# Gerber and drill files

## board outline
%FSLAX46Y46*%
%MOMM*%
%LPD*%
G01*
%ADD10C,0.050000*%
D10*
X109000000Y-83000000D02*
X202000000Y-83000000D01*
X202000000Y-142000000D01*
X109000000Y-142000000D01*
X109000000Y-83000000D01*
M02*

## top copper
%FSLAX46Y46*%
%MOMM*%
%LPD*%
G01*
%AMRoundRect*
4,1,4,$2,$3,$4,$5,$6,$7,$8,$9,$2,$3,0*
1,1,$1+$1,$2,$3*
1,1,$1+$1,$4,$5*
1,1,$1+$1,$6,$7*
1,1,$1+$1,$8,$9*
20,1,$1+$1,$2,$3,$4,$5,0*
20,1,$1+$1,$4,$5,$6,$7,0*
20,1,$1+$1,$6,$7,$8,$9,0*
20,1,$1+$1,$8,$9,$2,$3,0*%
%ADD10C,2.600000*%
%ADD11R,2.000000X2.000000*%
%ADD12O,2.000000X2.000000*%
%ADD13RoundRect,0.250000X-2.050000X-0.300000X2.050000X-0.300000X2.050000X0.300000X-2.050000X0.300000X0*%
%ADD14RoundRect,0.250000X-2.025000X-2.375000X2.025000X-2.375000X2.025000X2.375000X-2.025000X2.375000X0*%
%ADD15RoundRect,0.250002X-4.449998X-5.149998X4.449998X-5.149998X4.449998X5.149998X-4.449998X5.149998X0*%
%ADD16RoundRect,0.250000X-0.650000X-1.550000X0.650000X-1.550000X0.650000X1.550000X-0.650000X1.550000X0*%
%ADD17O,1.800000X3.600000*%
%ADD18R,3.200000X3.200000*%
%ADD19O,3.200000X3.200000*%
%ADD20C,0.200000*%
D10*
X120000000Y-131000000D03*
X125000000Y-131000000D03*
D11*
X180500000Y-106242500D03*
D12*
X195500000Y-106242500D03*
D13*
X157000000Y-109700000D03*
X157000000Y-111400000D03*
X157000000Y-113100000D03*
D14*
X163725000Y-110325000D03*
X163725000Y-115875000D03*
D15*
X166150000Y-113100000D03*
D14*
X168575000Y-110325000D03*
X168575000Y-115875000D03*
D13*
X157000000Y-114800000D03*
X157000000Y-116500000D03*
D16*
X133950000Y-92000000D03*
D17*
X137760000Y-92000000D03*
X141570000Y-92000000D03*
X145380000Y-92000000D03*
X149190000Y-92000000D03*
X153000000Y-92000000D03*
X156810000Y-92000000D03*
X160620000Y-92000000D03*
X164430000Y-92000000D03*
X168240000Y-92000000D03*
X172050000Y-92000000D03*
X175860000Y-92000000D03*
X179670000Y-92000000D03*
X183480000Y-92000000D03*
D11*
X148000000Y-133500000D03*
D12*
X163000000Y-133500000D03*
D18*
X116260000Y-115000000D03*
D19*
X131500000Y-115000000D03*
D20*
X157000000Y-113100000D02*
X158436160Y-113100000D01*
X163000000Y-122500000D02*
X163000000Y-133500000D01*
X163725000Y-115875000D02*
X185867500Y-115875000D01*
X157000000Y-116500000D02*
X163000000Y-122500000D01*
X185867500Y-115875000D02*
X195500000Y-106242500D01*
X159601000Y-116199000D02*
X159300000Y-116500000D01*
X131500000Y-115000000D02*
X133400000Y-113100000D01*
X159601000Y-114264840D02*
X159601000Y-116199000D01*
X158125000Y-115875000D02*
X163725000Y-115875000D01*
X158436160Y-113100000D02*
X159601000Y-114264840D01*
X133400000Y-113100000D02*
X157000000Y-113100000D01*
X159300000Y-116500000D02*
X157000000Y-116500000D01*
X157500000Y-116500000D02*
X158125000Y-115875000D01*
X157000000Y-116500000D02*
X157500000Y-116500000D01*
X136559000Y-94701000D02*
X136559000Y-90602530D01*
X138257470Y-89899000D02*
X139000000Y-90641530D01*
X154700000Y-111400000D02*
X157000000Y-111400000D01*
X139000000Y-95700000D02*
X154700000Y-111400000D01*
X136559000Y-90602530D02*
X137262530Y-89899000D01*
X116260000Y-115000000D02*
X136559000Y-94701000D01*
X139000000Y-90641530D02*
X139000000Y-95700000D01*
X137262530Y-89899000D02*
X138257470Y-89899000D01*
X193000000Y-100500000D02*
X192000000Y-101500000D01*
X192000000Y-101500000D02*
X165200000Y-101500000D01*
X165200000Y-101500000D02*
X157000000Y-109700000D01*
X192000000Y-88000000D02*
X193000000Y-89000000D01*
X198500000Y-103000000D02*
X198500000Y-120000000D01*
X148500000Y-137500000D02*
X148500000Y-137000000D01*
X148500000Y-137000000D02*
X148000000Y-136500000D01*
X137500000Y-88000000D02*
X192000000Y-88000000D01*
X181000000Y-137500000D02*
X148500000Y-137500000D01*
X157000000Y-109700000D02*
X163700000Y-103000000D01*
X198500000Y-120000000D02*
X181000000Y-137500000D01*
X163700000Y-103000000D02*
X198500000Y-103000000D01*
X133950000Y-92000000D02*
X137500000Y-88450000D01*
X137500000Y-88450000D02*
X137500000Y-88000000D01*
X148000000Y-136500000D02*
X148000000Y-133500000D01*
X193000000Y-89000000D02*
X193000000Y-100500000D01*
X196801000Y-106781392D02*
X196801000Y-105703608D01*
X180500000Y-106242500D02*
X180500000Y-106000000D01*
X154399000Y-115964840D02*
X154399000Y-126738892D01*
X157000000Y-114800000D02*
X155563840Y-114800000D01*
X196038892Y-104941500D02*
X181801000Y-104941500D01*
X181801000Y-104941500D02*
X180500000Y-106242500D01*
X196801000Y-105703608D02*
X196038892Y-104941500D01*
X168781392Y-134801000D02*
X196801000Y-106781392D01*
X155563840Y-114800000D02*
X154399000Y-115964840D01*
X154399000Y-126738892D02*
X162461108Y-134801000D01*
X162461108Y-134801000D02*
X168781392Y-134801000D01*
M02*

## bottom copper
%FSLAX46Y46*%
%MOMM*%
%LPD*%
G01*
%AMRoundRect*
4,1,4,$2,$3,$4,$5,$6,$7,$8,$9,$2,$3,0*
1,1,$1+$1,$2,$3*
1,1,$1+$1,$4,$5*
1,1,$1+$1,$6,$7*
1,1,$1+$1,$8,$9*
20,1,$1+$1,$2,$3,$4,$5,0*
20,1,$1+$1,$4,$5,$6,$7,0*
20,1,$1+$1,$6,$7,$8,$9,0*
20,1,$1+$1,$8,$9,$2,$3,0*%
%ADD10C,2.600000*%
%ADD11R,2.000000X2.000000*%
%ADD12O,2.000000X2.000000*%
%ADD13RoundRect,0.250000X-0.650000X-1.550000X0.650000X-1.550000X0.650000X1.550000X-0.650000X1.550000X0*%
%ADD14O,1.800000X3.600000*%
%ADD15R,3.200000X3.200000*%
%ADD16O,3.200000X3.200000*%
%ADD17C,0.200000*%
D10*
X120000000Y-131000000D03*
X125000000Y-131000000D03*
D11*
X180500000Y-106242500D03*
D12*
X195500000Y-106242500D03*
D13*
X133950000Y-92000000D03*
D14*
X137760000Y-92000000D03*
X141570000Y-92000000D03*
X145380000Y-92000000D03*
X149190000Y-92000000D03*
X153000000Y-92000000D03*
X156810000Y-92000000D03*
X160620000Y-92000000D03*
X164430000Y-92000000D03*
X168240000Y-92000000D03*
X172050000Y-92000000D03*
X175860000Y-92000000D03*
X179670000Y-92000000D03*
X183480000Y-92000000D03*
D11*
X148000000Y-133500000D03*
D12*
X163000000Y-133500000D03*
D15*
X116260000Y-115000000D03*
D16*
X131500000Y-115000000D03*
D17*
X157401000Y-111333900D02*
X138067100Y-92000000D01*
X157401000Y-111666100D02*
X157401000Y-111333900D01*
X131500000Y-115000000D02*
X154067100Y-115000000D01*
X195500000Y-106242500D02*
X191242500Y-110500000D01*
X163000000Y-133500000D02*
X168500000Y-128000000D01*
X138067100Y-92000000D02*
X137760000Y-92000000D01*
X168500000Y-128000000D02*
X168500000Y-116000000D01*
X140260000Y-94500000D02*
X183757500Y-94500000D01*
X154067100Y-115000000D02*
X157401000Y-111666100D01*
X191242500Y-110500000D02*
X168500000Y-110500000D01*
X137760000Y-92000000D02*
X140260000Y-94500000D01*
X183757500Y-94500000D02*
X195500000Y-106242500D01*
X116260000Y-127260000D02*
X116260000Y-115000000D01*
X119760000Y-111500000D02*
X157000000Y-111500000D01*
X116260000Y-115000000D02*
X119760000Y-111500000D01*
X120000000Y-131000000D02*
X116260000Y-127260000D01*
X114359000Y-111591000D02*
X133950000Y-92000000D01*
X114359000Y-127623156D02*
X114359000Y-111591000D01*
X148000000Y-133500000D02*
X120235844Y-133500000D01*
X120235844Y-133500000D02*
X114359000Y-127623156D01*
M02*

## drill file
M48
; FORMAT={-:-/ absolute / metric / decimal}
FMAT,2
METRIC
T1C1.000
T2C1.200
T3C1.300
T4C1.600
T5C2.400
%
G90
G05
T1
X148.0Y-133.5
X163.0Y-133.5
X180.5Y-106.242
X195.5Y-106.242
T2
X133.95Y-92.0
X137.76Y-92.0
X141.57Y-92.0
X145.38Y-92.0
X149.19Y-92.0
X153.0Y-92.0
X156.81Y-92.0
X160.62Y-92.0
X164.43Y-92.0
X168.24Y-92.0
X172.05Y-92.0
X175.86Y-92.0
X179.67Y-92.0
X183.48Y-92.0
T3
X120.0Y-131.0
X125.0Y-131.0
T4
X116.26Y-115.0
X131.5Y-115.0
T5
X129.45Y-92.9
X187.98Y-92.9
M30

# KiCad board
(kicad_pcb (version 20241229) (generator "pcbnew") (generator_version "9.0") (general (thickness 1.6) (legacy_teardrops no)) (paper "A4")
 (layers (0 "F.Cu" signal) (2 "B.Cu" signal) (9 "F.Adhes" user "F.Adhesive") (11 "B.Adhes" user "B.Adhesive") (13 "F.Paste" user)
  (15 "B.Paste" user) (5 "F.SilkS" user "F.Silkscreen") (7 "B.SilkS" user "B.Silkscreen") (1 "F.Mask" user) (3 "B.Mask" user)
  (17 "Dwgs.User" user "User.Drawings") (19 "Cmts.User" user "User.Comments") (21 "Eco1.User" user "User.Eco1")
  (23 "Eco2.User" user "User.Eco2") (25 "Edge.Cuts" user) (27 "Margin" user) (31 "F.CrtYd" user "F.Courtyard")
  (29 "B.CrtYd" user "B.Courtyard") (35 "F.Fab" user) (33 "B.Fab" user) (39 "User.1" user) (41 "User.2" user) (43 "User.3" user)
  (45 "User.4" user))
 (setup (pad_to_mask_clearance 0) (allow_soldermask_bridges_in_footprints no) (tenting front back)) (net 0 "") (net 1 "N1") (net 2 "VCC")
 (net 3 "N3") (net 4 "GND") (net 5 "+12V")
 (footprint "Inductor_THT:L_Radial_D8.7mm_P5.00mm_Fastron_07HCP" (layer "F.Cu") (at 120 131)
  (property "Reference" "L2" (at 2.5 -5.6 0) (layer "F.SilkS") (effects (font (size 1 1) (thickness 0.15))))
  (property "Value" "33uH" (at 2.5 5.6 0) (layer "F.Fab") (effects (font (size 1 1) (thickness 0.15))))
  (pad "1" thru_hole circle (at 0 0) (size 2.6 2.6) (drill 1.3) (layers "*.Cu" "*.Mask") (remove_unused_layers no) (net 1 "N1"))
  (pad "2" thru_hole circle (at 5 0) (size 2.6 2.6) (drill 1.3) (layers "*.Cu" "*.Mask") (remove_unused_layers no) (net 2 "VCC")))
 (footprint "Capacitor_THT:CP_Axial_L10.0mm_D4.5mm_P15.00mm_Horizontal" (layer "F.Cu") (at 180.5 106.2425)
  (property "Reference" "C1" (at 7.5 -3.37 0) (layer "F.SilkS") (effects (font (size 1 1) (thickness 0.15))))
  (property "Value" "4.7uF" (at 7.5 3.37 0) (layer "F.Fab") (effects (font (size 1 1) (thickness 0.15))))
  (pad "1" thru_hole rect (at 0 0) (size 2 2) (drill 1) (layers "*.Cu" "*.Mask") (remove_unused_layers no) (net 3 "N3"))
  (pad "2" thru_hole oval (at 15 0) (size 2 2) (drill 1) (layers "*.Cu" "*.Mask") (remove_unused_layers no) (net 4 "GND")))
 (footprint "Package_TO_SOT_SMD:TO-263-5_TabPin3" (layer "F.Cu") (at 164.65 113.1)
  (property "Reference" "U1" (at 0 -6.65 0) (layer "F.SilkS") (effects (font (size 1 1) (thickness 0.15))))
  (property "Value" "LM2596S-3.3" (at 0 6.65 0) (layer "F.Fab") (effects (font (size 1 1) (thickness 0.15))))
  (pad "1" smd roundrect (at -7.65 -3.4) (size 4.6 1.1) (layers "F.Cu" "F.Mask" "F.Paste") (roundrect_rratio 0.227273) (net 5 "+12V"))
  (pad "2" smd roundrect (at -7.65 -1.7) (size 4.6 1.1) (layers "F.Cu" "F.Mask" "F.Paste") (roundrect_rratio 0.227273) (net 1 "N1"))
  (pad "3" smd roundrect (at -7.65 0) (size 4.6 1.1) (layers "F.Cu" "F.Mask" "F.Paste") (roundrect_rratio 0.227273) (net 4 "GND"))
  (pad "3" smd roundrect (at -0.925 -2.775) (size 4.55 5.25) (layers "F.Cu" "F.Paste") (roundrect_rratio 0.054945) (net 4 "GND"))
  (pad "3" smd roundrect (at -0.925 2.775) (size 4.55 5.25) (layers "F.Cu" "F.Paste") (roundrect_rratio 0.054945) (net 4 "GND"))
  (pad "3" smd roundrect (at 1.5 0) (size 9.4 10.8) (layers "F.Cu" "F.Mask") (roundrect_rratio 0.026596) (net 4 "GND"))
  (pad "3" smd roundrect (at 3.925 -2.775) (size 4.55 5.25) (layers "F.Cu" "F.Paste") (roundrect_rratio 0.054945) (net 4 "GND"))
  (pad "3" smd roundrect (at 3.925 2.775) (size 4.55 5.25) (layers "F.Cu" "F.Paste") (roundrect_rratio 0.054945) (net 4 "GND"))
  (pad "4" smd roundrect (at -7.65 1.7) (size 4.6 1.1) (layers "F.Cu" "F.Mask" "F.Paste") (roundrect_rratio 0.227273) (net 3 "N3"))
  (pad "5" smd roundrect (at -7.65 3.4) (size 4.6 1.1) (layers "F.Cu" "F.Mask" "F.Paste") (roundrect_rratio 0.227273) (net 4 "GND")))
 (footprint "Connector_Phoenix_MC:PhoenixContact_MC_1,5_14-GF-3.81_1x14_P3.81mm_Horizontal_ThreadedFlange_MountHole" (layer "F.Cu")
  (at 133.95 92)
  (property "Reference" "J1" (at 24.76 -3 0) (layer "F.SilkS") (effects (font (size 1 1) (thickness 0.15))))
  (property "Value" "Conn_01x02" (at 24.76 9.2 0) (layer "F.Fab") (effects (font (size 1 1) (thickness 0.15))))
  (pad "" np_thru_hole circle (at -4.5 0.9) (size 2.4 2.4) (drill 2.4) (layers "*.Cu" "*.Mask"))
  (pad "" np_thru_hole circle (at 54.03 0.9) (size 2.4 2.4) (drill 2.4) (layers "*.Cu" "*.Mask"))
  (pad "1" thru_hole roundrect (at 0 0) (size 1.8 3.6) (drill 1.2) (layers "*.Cu" "*.Mask") (remove_unused_layers no)
   (roundrect_rratio 0.138889) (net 5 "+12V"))
  (pad "2" thru_hole oval (at 3.81 0) (size 1.8 3.6) (drill 1.2) (layers "*.Cu" "*.Mask") (remove_unused_layers no) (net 4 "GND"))
  (pad "3" thru_hole oval (at 7.62 0) (size 1.8 3.6) (drill 1.2) (layers "*.Cu" "*.Mask") (remove_unused_layers no))
  (pad "4" thru_hole oval (at 11.43 0) (size 1.8 3.6) (drill 1.2) (layers "*.Cu" "*.Mask") (remove_unused_layers no))
  (pad "5" thru_hole oval (at 15.24 0) (size 1.8 3.6) (drill 1.2) (layers "*.Cu" "*.Mask") (remove_unused_layers no))
  (pad "6" thru_hole oval (at 19.05 0) (size 1.8 3.6) (drill 1.2) (layers "*.Cu" "*.Mask") (remove_unused_layers no))
  (pad "7" thru_hole oval (at 22.86 0) (size 1.8 3.6) (drill 1.2) (layers "*.Cu" "*.Mask") (remove_unused_layers no))
  (pad "8" thru_hole oval (at 26.67 0) (size 1.8 3.6) (drill 1.2) (layers "*.Cu" "*.Mask") (remove_unused_layers no))
  (pad "9" thru_hole oval (at 30.48 0) (size 1.8 3.6) (drill 1.2) (layers "*.Cu" "*.Mask") (remove_unused_layers no))
  (pad "10" thru_hole oval (at 34.29 0) (size 1.8 3.6) (drill 1.2) (layers "*.Cu" "*.Mask") (remove_unused_layers no))
  (pad "11" thru_hole oval (at 38.1 0) (size 1.8 3.6) (drill 1.2) (layers "*.Cu" "*.Mask") (remove_unused_layers no))
  (pad "12" thru_hole oval (at 41.91 0) (size 1.8 3.6) (drill 1.2) (layers "*.Cu" "*.Mask") (remove_unused_layers no))
  (pad "13" thru_hole oval (at 45.72 0) (size 1.8 3.6) (drill 1.2) (layers "*.Cu" "*.Mask") (remove_unused_layers no))
  (pad "14" thru_hole oval (at 49.53 0) (size 1.8 3.6) (drill 1.2) (layers "*.Cu" "*.Mask") (remove_unused_layers no)))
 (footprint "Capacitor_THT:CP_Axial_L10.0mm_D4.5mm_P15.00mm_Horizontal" (layer "F.Cu") (at 148 133.5)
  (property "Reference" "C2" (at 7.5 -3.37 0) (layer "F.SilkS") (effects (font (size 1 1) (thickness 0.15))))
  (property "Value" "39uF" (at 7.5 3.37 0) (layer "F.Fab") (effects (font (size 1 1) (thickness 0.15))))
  (pad "1" thru_hole rect (at 0 0) (size 2 2) (drill 1) (layers "*.Cu" "*.Mask") (remove_unused_layers no) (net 5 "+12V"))
  (pad "2" thru_hole oval (at 15 0) (size 2 2) (drill 1) (layers "*.Cu" "*.Mask") (remove_unused_layers no) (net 4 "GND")))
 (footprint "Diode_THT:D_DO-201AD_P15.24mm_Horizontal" (layer "F.Cu") (at 116.26 115)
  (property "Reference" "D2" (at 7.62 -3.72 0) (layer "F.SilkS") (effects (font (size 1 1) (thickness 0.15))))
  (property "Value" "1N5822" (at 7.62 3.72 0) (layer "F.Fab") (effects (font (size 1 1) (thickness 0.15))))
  (pad "1" thru_hole rect (at 0 0) (size 3.2 3.2) (drill 1.6) (layers "*.Cu" "*.Mask") (remove_unused_layers no) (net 1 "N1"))
  (pad "2" thru_hole oval (at 15.24 0) (size 3.2 3.2) (drill 1.6) (layers "*.Cu" "*.Mask") (remove_unused_layers no) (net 4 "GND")))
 (gr_rect (start 109 83) (end 202 142) (stroke (width 0.05) (type default)) (fill no) (layer "Edge.Cuts"))
 (segment (start 157 113.1) (end 158.43616 113.1) (width 0.2) (layer "F.Cu") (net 4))
 (segment (start 163 122.5) (end 163 133.5) (width 0.2) (layer "F.Cu") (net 4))
 (segment (start 163.725 115.875) (end 185.8675 115.875) (width 0.2) (layer "F.Cu") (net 4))
 (segment (start 157 116.5) (end 163 122.5) (width 0.2) (layer "F.Cu") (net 4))
 (segment (start 185.8675 115.875) (end 195.5 106.2425) (width 0.2) (layer "F.Cu") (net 4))
 (segment (start 159.601 116.199) (end 159.3 116.5) (width 0.2) (layer "F.Cu") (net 4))
 (segment (start 131.5 115) (end 133.4 113.1) (width 0.2) (layer "F.Cu") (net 4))
 (segment (start 159.601 114.26484) (end 159.601 116.199) (width 0.2) (layer "F.Cu") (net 4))
 (segment (start 158.125 115.875) (end 163.725 115.875) (width 0.2) (layer "F.Cu") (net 4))
 (segment (start 158.43616 113.1) (end 159.601 114.26484) (width 0.2) (layer "F.Cu") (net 4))
 (segment (start 133.4 113.1) (end 157 113.1) (width 0.2) (layer "F.Cu") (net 4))
 (segment (start 159.3 116.5) (end 157 116.5) (width 0.2) (layer "F.Cu") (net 4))
 (segment (start 157.5 116.5) (end 158.125 115.875) (width 0.2) (layer "F.Cu") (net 4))
 (segment (start 157 116.5) (end 157.5 116.5) (width 0.2) (layer "F.Cu") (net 4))
 (segment (start 157.401 111.3339) (end 138.0671 92) (width 0.2) (layer "B.Cu") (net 4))
 (segment (start 157.401 111.6661) (end 157.401 111.3339) (width 0.2) (layer "B.Cu") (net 4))
 (segment (start 131.5 115) (end 154.0671 115) (width 0.2) (layer "B.Cu") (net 4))
 (segment (start 195.5 106.2425) (end 191.2425 110.5) (width 0.2) (layer "B.Cu") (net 4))
 (segment (start 163 133.5) (end 168.5 128) (width 0.2) (layer "B.Cu") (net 4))
 (segment (start 138.0671 92) (end 137.76 92) (width 0.2) (layer "B.Cu") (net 4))
 (segment (start 168.5 128) (end 168.5 116) (width 0.2) (layer "B.Cu") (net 4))
 (segment (start 140.26 94.5) (end 183.7575 94.5) (width 0.2) (layer "B.Cu") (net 4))
 (segment (start 154.0671 115) (end 157.401 111.6661) (width 0.2) (layer "B.Cu") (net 4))
 (segment (start 191.2425 110.5) (end 168.5 110.5) (width 0.2) (layer "B.Cu") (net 4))
 (segment (start 137.76 92) (end 140.26 94.5) (width 0.2) (layer "B.Cu") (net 4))
 (segment (start 183.7575 94.5) (end 195.5 106.2425) (width 0.2) (layer "B.Cu") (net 4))
 (segment (start 136.559 94.701) (end 136.559 90.60253) (width 0.2) (layer "F.Cu") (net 1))
 (segment (start 138.25747 89.899) (end 139 90.64153) (width 0.2) (layer "F.Cu") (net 1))
 (segment (start 154.7 111.4) (end 157 111.4) (width 0.2) (layer "F.Cu") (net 1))
 (segment (start 139 95.7) (end 154.7 111.4) (width 0.2) (layer "F.Cu") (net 1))
 (segment (start 136.559 90.60253) (end 137.26253 89.899) (width 0.2) (layer "F.Cu") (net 1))
 (segment (start 116.26 115) (end 136.559 94.701) (width 0.2) (layer "F.Cu") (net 1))
 (segment (start 139 90.64153) (end 139 95.7) (width 0.2) (layer "F.Cu") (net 1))
 (segment (start 137.26253 89.899) (end 138.25747 89.899) (width 0.2) (layer "F.Cu") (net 1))
 (segment (start 116.26 127.26) (end 116.26 115) (width 0.2) (layer "B.Cu") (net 1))
 (segment (start 119.76 111.5) (end 157 111.5) (width 0.2) (layer "B.Cu") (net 1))
 (segment (start 116.26 115) (end 119.76 111.5) (width 0.2) (layer "B.Cu") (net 1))
 (segment (start 120 131) (end 116.26 127.26) (width 0.2) (layer "B.Cu") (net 1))
 (segment (start 193 100.5) (end 192 101.5) (width 0.2) (layer "F.Cu") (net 5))
 (segment (start 192 101.5) (end 165.2 101.5) (width 0.2) (layer "F.Cu") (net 5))
 (segment (start 165.2 101.5) (end 157 109.7) (width 0.2) (layer "F.Cu") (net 5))
 (segment (start 192 88) (end 193 89) (width 0.2) (layer "F.Cu") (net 5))
 (segment (start 198.5 103) (end 198.5 120) (width 0.2) (layer "F.Cu") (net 5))
 (segment (start 148.5 137.5) (end 148.5 137) (width 0.2) (layer "F.Cu") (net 5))
 (segment (start 148.5 137) (end 148 136.5) (width 0.2) (layer "F.Cu") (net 5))
 (segment (start 137.5 88) (end 192 88) (width 0.2) (layer "F.Cu") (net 5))
 (segment (start 181 137.5) (end 148.5 137.5) (width 0.2) (layer "F.Cu") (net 5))
 (segment (start 157 109.7) (end 163.7 103) (width 0.2) (layer "F.Cu") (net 5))
 (segment (start 198.5 120) (end 181 137.5) (width 0.2) (layer "F.Cu") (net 5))
 (segment (start 163.7 103) (end 198.5 103) (width 0.2) (layer "F.Cu") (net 5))
 (segment (start 133.95 92) (end 137.5 88.45) (width 0.2) (layer "F.Cu") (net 5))
 (segment (start 137.5 88.45) (end 137.5 88) (width 0.2) (layer "F.Cu") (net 5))
 (segment (start 148 136.5) (end 148 133.5) (width 0.2) (layer "F.Cu") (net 5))
 (segment (start 193 89) (end 193 100.5) (width 0.2) (layer "F.Cu") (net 5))
 (segment (start 114.359 111.591) (end 133.95 92) (width 0.2) (layer "B.Cu") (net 5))
 (segment (start 114.359 127.623156) (end 114.359 111.591) (width 0.2) (layer "B.Cu") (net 5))
 (segment (start 148 133.5) (end 120.235844 133.5) (width 0.2) (layer "B.Cu") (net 5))
 (segment (start 120.235844 133.5) (end 114.359 127.623156) (width 0.2) (layer "B.Cu") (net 5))
 (segment (start 196.801 106.781392) (end 196.801 105.703608) (width 0.2) (layer "F.Cu") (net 3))
 (segment (start 180.5 106.2425) (end 180.5 106) (width 0.2) (layer "F.Cu") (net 3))
 (segment (start 154.399 115.96484) (end 154.399 126.738892) (width 0.2) (layer "F.Cu") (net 3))
 (segment (start 157 114.8) (end 155.56384 114.8) (width 0.2) (layer "F.Cu") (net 3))
 (segment (start 196.038892 104.9415) (end 181.801 104.9415) (width 0.2) (layer "F.Cu") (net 3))
 (segment (start 181.801 104.9415) (end 180.5 106.2425) (width 0.2) (layer "F.Cu") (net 3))
 (segment (start 196.801 105.703608) (end 196.038892 104.9415) (width 0.2) (layer "F.Cu") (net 3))
 (segment (start 168.781392 134.801) (end 196.801 106.781392) (width 0.2) (layer "F.Cu") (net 3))
 (segment (start 155.56384 114.8) (end 154.399 115.96484) (width 0.2) (layer "F.Cu") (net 3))
 (segment (start 154.399 126.738892) (end 162.461108 134.801) (width 0.2) (layer "F.Cu") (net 3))
 (segment (start 162.461108 134.801) (end 168.781392 134.801) (width 0.2) (layer "F.Cu") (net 3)))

